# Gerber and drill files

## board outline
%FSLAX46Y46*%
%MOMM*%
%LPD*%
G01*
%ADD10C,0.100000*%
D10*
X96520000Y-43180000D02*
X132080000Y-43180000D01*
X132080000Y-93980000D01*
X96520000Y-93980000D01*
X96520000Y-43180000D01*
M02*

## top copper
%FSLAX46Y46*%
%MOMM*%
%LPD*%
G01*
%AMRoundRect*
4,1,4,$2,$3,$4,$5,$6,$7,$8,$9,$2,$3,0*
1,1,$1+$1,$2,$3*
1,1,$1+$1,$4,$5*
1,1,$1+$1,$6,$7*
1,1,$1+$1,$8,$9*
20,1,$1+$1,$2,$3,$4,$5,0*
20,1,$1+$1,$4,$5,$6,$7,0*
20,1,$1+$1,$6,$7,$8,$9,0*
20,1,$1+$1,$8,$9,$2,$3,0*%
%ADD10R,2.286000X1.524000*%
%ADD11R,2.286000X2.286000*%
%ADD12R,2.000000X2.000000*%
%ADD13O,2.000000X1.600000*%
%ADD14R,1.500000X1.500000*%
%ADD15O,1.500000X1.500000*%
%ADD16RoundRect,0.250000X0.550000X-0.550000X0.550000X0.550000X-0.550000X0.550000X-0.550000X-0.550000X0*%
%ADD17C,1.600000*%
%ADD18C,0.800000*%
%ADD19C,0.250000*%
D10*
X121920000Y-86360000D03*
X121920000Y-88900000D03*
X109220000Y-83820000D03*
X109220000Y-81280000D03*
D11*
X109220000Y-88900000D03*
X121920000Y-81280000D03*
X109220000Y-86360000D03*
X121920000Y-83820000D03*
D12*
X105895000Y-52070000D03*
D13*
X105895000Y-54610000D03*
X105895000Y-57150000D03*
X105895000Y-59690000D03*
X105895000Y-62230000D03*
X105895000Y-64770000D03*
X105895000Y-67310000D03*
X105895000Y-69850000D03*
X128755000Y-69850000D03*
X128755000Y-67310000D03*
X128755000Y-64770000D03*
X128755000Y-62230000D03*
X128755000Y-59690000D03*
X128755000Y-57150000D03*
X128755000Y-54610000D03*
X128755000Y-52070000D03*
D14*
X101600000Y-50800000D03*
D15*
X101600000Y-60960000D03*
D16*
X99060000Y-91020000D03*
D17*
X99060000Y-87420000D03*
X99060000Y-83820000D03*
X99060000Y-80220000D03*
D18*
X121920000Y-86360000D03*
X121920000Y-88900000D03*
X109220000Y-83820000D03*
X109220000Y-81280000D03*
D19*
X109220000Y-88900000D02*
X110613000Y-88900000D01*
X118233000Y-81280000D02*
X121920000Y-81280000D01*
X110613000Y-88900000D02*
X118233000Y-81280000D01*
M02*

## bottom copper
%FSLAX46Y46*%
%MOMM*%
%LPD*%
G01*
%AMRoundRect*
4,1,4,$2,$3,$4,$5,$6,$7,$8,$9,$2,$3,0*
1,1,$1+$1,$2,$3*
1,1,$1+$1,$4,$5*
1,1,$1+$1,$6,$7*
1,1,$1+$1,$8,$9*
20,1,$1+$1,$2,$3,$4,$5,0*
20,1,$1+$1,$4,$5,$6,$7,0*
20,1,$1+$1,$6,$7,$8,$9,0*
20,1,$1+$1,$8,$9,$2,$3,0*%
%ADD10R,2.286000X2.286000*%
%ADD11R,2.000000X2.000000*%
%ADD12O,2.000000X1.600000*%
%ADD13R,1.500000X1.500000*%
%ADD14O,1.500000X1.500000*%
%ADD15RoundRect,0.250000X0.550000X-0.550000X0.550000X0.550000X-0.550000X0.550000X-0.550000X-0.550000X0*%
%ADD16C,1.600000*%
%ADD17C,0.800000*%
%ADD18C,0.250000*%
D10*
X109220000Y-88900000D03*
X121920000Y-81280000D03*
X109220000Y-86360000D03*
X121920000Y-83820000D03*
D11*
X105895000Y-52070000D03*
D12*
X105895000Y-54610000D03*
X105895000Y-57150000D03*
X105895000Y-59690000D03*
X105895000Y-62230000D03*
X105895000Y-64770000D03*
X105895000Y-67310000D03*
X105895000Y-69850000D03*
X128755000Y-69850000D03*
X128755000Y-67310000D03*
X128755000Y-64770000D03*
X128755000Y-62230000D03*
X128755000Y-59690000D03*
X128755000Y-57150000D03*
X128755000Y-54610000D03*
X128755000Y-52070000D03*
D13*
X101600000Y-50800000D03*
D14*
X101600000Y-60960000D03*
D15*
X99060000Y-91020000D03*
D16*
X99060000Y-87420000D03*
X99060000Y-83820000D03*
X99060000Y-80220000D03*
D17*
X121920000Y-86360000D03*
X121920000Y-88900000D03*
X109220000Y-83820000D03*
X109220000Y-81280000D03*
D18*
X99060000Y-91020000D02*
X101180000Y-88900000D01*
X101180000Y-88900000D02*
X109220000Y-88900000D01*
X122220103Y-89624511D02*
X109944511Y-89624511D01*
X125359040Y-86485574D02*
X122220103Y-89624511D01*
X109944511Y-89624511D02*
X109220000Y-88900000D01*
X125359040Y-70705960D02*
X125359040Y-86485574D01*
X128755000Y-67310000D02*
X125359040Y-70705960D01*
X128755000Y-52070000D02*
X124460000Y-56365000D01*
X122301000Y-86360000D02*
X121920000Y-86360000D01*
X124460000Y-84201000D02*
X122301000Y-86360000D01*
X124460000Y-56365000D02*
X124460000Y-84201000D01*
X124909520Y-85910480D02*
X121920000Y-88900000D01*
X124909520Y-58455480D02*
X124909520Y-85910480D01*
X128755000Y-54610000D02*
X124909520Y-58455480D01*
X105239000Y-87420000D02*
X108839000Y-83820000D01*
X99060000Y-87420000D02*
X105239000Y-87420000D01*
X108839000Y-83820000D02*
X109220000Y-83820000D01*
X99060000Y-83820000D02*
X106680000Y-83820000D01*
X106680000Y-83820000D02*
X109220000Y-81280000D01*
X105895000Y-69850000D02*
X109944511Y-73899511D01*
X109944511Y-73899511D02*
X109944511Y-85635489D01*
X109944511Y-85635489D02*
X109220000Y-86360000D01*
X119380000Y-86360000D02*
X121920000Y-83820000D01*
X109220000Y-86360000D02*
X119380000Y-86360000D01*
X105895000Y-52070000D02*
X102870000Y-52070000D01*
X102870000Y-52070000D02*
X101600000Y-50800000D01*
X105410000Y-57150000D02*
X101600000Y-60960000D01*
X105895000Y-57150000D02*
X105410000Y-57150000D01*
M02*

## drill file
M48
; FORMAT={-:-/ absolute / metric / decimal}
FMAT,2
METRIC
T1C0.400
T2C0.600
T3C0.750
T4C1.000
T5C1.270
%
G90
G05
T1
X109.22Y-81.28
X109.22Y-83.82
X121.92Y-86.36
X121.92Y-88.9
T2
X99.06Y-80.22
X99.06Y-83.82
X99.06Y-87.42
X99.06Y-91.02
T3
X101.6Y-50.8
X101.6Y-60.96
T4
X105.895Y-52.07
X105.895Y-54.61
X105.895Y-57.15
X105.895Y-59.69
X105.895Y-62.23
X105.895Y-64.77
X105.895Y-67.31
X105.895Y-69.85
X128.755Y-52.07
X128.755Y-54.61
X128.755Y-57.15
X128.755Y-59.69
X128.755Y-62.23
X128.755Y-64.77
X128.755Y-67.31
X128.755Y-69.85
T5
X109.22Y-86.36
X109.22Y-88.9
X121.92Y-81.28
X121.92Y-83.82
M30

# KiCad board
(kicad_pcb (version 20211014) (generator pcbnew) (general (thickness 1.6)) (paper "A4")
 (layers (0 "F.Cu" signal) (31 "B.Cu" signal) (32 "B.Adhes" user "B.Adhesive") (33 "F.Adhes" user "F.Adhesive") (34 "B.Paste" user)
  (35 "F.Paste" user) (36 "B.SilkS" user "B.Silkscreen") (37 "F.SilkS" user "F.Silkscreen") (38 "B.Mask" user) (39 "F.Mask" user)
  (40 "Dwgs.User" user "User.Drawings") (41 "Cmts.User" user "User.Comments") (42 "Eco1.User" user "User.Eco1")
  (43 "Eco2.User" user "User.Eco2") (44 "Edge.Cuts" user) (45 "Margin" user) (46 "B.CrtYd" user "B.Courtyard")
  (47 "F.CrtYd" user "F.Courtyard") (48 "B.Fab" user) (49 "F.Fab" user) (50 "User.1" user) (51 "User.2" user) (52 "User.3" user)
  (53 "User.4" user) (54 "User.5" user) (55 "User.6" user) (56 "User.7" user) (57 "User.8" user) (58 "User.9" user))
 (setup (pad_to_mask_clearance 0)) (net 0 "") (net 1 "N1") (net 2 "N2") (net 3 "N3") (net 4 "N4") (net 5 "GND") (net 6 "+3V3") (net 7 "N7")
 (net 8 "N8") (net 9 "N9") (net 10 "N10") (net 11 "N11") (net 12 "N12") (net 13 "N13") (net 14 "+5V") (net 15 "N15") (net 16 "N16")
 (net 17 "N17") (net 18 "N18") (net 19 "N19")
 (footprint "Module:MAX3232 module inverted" (layer "F.Cu") (at 116.84 83.82)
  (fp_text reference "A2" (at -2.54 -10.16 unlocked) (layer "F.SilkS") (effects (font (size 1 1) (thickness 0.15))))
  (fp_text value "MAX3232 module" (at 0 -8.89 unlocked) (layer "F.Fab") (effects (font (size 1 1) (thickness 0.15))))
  (pad "11" smd rect (at 5.08 2.54) (size 2.286 1.524) (layers "F.Cu" "F.Paste" "F.Mask") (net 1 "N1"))
  (pad "12" smd rect (at 5.08 5.08) (size 2.286 1.524) (layers "F.Cu" "F.Paste" "F.Mask") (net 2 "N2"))
  (pad "13" smd rect (at -7.62 0) (size 2.286 1.524) (layers "F.Cu" "F.Paste" "F.Mask") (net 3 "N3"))
  (pad "14" smd rect (at -7.62 -2.54) (size 2.286 1.524) (layers "F.Cu" "F.Paste" "F.Mask") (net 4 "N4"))
  (pad "15" thru_hole rect (at -7.62 5.08) (size 2.286 2.286) (drill 1.27) (layers *.Cu *.Mask) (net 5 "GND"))
  (pad "15" thru_hole rect (at 5.08 -2.54) (size 2.286 2.286) (drill 1.27) (layers *.Cu *.Mask) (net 5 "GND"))
  (pad "16" thru_hole rect (at -7.62 2.54) (size 2.286 2.286) (drill 1.27) (layers *.Cu *.Mask) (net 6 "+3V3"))
  (pad "16" thru_hole rect (at 5.08 0) (size 2.286 2.286) (drill 1.27) (layers *.Cu *.Mask) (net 6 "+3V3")))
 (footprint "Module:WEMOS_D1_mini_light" (layer "F.Cu") (at 105.895 52.07)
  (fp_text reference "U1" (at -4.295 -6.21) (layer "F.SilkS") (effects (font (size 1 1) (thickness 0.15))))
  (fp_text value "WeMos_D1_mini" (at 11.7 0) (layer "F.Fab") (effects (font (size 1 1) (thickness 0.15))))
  (pad "1" thru_hole rect (at 0 0) (size 2 2) (drill 1) (layers *.Cu *.Mask) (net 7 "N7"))
  (pad "2" thru_hole oval (at 0 2.54) (size 2 1.6) (drill 1) (layers *.Cu *.Mask) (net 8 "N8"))
  (pad "3" thru_hole oval (at 0 5.08) (size 2 1.6) (drill 1) (layers *.Cu *.Mask) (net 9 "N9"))
  (pad "4" thru_hole oval (at 0 7.62) (size 2 1.6) (drill 1) (layers *.Cu *.Mask) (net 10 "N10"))
  (pad "5" thru_hole oval (at 0 10.16) (size 2 1.6) (drill 1) (layers *.Cu *.Mask) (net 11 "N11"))
  (pad "6" thru_hole oval (at 0 12.7) (size 2 1.6) (drill 1) (layers *.Cu *.Mask) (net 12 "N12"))
  (pad "7" thru_hole oval (at 0 15.24) (size 2 1.6) (drill 1) (layers *.Cu *.Mask) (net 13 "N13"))
  (pad "8" thru_hole oval (at 0 17.78) (size 2 1.6) (drill 1) (layers *.Cu *.Mask) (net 6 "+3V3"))
  (pad "9" thru_hole oval (at 22.86 17.78) (size 2 1.6) (drill 1) (layers *.Cu *.Mask) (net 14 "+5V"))
  (pad "10" thru_hole oval (at 22.86 15.24) (size 2 1.6) (drill 1) (layers *.Cu *.Mask) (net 5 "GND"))
  (pad "11" thru_hole oval (at 22.86 12.7) (size 2 1.6) (drill 1) (layers *.Cu *.Mask) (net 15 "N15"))
  (pad "12" thru_hole oval (at 22.86 10.16) (size 2 1.6) (drill 1) (layers *.Cu *.Mask) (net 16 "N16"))
  (pad "13" thru_hole oval (at 22.86 7.62) (size 2 1.6) (drill 1) (layers *.Cu *.Mask) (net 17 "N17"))
  (pad "14" thru_hole oval (at 22.86 5.08) (size 2 1.6) (drill 1) (layers *.Cu *.Mask) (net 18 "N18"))
  (pad "15" thru_hole oval (at 22.86 2.54) (size 2 1.6) (drill 1) (layers *.Cu *.Mask) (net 2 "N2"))
  (pad "16" thru_hole oval (at 22.86 0) (size 2 1.6) (drill 1) (layers *.Cu *.Mask) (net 1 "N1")))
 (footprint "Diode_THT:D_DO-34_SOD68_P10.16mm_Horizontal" (layer "F.Cu") (at 101.6 50.8 -90)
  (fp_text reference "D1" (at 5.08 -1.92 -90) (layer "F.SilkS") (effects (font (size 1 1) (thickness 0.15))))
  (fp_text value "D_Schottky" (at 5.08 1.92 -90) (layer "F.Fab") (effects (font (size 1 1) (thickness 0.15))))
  (pad "1" thru_hole rect (at 0 0 270) (size 1.5 1.5) (drill 0.75) (layers *.Cu *.Mask) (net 7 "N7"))
  (pad "2" thru_hole oval (at 10.16 0 270) (size 1.5 1.5) (drill 0.75) (layers *.Cu *.Mask) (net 9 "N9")))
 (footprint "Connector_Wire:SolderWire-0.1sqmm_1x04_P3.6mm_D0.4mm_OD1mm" (layer "F.Cu") (at 99.06 91.02 90)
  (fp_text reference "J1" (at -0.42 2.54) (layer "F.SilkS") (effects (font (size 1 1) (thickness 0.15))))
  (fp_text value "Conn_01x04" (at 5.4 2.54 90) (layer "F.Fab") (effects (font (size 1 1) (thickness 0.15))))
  (pad "1" thru_hole roundrect (at 0 0 90) (size 1.6 1.6) (drill 0.6) (layers *.Cu *.Mask) (roundrect_rratio 0.15625) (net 5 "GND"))
  (pad "2" thru_hole circle (at 3.6 0 90) (size 1.6 1.6) (drill 0.6) (layers *.Cu *.Mask) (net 3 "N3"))
  (pad "3" thru_hole circle (at 7.2 0 90) (size 1.6 1.6) (drill 0.6) (layers *.Cu *.Mask) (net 4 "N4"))
  (pad "4" thru_hole circle (at 10.8 0 90) (size 1.6 1.6) (drill 0.6) (layers *.Cu *.Mask) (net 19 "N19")))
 (gr_rect (start 132.08 43.18) (end 96.52 93.98) (layer "Edge.Cuts") (width 0.1) (fill none))
 (segment (start 109.22 88.9) (end 110.613 88.9) (width 0.25) (layer "F.Cu") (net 5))
 (segment (start 118.233 81.28) (end 121.92 81.28) (width 0.25) (layer "F.Cu") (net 5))
 (segment (start 110.613 88.9) (end 118.233 81.28) (width 0.25) (layer "F.Cu") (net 5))
 (segment (start 99.06 91.02) (end 101.18 88.9) (width 0.25) (layer "B.Cu") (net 5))
 (segment (start 101.18 88.9) (end 109.22 88.9) (width 0.25) (layer "B.Cu") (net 5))
 (segment (start 122.220103 89.624511) (end 109.944511 89.624511) (width 0.25) (layer "B.Cu") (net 5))
 (segment (start 125.35904 86.485574) (end 122.220103 89.624511) (width 0.25) (layer "B.Cu") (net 5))
 (segment (start 109.944511 89.624511) (end 109.22 88.9) (width 0.25) (layer "B.Cu") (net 5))
 (segment (start 125.35904 70.70596) (end 125.35904 86.485574) (width 0.25) (layer "B.Cu") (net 5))
 (segment (start 128.755 67.31) (end 125.35904 70.70596) (width 0.25) (layer "B.Cu") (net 5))
 (via (at 121.92 86.36) (size 0.8) (drill 0.4) (layers "F.Cu" "B.Cu") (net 1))
 (segment (start 128.755 52.07) (end 124.46 56.365) (width 0.25) (layer "B.Cu") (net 1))
 (segment (start 122.301 86.36) (end 121.92 86.36) (width 0.25) (layer "B.Cu") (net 1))
 (segment (start 124.46 84.201) (end 122.301 86.36) (width 0.25) (layer "B.Cu") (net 1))
 (segment (start 124.46 56.365) (end 124.46 84.201) (width 0.25) (layer "B.Cu") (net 1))
 (via (at 121.92 88.9) (size 0.8) (drill 0.4) (layers "F.Cu" "B.Cu") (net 2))
 (segment (start 124.90952 85.91048) (end 121.92 88.9) (width 0.25) (layer "B.Cu") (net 2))
 (segment (start 124.90952 58.45548) (end 124.90952 85.91048) (width 0.25) (layer "B.Cu") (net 2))
 (segment (start 128.755 54.61) (end 124.90952 58.45548) (width 0.25) (layer "B.Cu") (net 2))
 (via (at 109.22 83.82) (size 0.8) (drill 0.4) (layers "F.Cu" "B.Cu") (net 3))
 (segment (start 105.239 87.42) (end 108.839 83.82) (width 0.25) (layer "B.Cu") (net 3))
 (segment (start 99.06 87.42) (end 105.239 87.42) (width 0.25) (layer "B.Cu") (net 3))
 (segment (start 108.839 83.82) (end 109.22 83.82) (width 0.25) (layer "B.Cu") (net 3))
 (via (at 109.22 81.28) (size 0.8) (drill 0.4) (layers "F.Cu" "B.Cu") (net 4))
 (segment (start 99.06 83.82) (end 106.68 83.82) (width 0.25) (layer "B.Cu") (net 4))
 (segment (start 106.68 83.82) (end 109.22 81.28) (width 0.25) (layer "B.Cu") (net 4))
 (segment (start 105.895 69.85) (end 109.944511 73.899511) (width 0.25) (layer "B.Cu") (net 6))
 (segment (start 109.944511 73.899511) (end 109.944511 85.635489) (width 0.25) (layer "B.Cu") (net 6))
 (segment (start 109.944511 85.635489) (end 109.22 86.36) (width 0.25) (layer "B.Cu") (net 6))
 (segment (start 119.38 86.36) (end 121.92 83.82) (width 0.25) (layer "B.Cu") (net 6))
 (segment (start 109.22 86.36) (end 119.38 86.36) (width 0.25) (layer "B.Cu") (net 6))
 (segment (start 105.895 52.07) (end 102.87 52.07) (width 0.25) (layer "B.Cu") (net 7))
 (segment (start 102.87 52.07) (end 101.6 50.8) (width 0.25) (layer "B.Cu") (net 7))
 (segment (start 105.41 57.15) (end 101.6 60.96) (width 0.25) (layer "B.Cu") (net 9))
 (segment (start 105.895 57.15) (end 105.41 57.15) (width 0.25) (layer "B.Cu") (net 9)))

